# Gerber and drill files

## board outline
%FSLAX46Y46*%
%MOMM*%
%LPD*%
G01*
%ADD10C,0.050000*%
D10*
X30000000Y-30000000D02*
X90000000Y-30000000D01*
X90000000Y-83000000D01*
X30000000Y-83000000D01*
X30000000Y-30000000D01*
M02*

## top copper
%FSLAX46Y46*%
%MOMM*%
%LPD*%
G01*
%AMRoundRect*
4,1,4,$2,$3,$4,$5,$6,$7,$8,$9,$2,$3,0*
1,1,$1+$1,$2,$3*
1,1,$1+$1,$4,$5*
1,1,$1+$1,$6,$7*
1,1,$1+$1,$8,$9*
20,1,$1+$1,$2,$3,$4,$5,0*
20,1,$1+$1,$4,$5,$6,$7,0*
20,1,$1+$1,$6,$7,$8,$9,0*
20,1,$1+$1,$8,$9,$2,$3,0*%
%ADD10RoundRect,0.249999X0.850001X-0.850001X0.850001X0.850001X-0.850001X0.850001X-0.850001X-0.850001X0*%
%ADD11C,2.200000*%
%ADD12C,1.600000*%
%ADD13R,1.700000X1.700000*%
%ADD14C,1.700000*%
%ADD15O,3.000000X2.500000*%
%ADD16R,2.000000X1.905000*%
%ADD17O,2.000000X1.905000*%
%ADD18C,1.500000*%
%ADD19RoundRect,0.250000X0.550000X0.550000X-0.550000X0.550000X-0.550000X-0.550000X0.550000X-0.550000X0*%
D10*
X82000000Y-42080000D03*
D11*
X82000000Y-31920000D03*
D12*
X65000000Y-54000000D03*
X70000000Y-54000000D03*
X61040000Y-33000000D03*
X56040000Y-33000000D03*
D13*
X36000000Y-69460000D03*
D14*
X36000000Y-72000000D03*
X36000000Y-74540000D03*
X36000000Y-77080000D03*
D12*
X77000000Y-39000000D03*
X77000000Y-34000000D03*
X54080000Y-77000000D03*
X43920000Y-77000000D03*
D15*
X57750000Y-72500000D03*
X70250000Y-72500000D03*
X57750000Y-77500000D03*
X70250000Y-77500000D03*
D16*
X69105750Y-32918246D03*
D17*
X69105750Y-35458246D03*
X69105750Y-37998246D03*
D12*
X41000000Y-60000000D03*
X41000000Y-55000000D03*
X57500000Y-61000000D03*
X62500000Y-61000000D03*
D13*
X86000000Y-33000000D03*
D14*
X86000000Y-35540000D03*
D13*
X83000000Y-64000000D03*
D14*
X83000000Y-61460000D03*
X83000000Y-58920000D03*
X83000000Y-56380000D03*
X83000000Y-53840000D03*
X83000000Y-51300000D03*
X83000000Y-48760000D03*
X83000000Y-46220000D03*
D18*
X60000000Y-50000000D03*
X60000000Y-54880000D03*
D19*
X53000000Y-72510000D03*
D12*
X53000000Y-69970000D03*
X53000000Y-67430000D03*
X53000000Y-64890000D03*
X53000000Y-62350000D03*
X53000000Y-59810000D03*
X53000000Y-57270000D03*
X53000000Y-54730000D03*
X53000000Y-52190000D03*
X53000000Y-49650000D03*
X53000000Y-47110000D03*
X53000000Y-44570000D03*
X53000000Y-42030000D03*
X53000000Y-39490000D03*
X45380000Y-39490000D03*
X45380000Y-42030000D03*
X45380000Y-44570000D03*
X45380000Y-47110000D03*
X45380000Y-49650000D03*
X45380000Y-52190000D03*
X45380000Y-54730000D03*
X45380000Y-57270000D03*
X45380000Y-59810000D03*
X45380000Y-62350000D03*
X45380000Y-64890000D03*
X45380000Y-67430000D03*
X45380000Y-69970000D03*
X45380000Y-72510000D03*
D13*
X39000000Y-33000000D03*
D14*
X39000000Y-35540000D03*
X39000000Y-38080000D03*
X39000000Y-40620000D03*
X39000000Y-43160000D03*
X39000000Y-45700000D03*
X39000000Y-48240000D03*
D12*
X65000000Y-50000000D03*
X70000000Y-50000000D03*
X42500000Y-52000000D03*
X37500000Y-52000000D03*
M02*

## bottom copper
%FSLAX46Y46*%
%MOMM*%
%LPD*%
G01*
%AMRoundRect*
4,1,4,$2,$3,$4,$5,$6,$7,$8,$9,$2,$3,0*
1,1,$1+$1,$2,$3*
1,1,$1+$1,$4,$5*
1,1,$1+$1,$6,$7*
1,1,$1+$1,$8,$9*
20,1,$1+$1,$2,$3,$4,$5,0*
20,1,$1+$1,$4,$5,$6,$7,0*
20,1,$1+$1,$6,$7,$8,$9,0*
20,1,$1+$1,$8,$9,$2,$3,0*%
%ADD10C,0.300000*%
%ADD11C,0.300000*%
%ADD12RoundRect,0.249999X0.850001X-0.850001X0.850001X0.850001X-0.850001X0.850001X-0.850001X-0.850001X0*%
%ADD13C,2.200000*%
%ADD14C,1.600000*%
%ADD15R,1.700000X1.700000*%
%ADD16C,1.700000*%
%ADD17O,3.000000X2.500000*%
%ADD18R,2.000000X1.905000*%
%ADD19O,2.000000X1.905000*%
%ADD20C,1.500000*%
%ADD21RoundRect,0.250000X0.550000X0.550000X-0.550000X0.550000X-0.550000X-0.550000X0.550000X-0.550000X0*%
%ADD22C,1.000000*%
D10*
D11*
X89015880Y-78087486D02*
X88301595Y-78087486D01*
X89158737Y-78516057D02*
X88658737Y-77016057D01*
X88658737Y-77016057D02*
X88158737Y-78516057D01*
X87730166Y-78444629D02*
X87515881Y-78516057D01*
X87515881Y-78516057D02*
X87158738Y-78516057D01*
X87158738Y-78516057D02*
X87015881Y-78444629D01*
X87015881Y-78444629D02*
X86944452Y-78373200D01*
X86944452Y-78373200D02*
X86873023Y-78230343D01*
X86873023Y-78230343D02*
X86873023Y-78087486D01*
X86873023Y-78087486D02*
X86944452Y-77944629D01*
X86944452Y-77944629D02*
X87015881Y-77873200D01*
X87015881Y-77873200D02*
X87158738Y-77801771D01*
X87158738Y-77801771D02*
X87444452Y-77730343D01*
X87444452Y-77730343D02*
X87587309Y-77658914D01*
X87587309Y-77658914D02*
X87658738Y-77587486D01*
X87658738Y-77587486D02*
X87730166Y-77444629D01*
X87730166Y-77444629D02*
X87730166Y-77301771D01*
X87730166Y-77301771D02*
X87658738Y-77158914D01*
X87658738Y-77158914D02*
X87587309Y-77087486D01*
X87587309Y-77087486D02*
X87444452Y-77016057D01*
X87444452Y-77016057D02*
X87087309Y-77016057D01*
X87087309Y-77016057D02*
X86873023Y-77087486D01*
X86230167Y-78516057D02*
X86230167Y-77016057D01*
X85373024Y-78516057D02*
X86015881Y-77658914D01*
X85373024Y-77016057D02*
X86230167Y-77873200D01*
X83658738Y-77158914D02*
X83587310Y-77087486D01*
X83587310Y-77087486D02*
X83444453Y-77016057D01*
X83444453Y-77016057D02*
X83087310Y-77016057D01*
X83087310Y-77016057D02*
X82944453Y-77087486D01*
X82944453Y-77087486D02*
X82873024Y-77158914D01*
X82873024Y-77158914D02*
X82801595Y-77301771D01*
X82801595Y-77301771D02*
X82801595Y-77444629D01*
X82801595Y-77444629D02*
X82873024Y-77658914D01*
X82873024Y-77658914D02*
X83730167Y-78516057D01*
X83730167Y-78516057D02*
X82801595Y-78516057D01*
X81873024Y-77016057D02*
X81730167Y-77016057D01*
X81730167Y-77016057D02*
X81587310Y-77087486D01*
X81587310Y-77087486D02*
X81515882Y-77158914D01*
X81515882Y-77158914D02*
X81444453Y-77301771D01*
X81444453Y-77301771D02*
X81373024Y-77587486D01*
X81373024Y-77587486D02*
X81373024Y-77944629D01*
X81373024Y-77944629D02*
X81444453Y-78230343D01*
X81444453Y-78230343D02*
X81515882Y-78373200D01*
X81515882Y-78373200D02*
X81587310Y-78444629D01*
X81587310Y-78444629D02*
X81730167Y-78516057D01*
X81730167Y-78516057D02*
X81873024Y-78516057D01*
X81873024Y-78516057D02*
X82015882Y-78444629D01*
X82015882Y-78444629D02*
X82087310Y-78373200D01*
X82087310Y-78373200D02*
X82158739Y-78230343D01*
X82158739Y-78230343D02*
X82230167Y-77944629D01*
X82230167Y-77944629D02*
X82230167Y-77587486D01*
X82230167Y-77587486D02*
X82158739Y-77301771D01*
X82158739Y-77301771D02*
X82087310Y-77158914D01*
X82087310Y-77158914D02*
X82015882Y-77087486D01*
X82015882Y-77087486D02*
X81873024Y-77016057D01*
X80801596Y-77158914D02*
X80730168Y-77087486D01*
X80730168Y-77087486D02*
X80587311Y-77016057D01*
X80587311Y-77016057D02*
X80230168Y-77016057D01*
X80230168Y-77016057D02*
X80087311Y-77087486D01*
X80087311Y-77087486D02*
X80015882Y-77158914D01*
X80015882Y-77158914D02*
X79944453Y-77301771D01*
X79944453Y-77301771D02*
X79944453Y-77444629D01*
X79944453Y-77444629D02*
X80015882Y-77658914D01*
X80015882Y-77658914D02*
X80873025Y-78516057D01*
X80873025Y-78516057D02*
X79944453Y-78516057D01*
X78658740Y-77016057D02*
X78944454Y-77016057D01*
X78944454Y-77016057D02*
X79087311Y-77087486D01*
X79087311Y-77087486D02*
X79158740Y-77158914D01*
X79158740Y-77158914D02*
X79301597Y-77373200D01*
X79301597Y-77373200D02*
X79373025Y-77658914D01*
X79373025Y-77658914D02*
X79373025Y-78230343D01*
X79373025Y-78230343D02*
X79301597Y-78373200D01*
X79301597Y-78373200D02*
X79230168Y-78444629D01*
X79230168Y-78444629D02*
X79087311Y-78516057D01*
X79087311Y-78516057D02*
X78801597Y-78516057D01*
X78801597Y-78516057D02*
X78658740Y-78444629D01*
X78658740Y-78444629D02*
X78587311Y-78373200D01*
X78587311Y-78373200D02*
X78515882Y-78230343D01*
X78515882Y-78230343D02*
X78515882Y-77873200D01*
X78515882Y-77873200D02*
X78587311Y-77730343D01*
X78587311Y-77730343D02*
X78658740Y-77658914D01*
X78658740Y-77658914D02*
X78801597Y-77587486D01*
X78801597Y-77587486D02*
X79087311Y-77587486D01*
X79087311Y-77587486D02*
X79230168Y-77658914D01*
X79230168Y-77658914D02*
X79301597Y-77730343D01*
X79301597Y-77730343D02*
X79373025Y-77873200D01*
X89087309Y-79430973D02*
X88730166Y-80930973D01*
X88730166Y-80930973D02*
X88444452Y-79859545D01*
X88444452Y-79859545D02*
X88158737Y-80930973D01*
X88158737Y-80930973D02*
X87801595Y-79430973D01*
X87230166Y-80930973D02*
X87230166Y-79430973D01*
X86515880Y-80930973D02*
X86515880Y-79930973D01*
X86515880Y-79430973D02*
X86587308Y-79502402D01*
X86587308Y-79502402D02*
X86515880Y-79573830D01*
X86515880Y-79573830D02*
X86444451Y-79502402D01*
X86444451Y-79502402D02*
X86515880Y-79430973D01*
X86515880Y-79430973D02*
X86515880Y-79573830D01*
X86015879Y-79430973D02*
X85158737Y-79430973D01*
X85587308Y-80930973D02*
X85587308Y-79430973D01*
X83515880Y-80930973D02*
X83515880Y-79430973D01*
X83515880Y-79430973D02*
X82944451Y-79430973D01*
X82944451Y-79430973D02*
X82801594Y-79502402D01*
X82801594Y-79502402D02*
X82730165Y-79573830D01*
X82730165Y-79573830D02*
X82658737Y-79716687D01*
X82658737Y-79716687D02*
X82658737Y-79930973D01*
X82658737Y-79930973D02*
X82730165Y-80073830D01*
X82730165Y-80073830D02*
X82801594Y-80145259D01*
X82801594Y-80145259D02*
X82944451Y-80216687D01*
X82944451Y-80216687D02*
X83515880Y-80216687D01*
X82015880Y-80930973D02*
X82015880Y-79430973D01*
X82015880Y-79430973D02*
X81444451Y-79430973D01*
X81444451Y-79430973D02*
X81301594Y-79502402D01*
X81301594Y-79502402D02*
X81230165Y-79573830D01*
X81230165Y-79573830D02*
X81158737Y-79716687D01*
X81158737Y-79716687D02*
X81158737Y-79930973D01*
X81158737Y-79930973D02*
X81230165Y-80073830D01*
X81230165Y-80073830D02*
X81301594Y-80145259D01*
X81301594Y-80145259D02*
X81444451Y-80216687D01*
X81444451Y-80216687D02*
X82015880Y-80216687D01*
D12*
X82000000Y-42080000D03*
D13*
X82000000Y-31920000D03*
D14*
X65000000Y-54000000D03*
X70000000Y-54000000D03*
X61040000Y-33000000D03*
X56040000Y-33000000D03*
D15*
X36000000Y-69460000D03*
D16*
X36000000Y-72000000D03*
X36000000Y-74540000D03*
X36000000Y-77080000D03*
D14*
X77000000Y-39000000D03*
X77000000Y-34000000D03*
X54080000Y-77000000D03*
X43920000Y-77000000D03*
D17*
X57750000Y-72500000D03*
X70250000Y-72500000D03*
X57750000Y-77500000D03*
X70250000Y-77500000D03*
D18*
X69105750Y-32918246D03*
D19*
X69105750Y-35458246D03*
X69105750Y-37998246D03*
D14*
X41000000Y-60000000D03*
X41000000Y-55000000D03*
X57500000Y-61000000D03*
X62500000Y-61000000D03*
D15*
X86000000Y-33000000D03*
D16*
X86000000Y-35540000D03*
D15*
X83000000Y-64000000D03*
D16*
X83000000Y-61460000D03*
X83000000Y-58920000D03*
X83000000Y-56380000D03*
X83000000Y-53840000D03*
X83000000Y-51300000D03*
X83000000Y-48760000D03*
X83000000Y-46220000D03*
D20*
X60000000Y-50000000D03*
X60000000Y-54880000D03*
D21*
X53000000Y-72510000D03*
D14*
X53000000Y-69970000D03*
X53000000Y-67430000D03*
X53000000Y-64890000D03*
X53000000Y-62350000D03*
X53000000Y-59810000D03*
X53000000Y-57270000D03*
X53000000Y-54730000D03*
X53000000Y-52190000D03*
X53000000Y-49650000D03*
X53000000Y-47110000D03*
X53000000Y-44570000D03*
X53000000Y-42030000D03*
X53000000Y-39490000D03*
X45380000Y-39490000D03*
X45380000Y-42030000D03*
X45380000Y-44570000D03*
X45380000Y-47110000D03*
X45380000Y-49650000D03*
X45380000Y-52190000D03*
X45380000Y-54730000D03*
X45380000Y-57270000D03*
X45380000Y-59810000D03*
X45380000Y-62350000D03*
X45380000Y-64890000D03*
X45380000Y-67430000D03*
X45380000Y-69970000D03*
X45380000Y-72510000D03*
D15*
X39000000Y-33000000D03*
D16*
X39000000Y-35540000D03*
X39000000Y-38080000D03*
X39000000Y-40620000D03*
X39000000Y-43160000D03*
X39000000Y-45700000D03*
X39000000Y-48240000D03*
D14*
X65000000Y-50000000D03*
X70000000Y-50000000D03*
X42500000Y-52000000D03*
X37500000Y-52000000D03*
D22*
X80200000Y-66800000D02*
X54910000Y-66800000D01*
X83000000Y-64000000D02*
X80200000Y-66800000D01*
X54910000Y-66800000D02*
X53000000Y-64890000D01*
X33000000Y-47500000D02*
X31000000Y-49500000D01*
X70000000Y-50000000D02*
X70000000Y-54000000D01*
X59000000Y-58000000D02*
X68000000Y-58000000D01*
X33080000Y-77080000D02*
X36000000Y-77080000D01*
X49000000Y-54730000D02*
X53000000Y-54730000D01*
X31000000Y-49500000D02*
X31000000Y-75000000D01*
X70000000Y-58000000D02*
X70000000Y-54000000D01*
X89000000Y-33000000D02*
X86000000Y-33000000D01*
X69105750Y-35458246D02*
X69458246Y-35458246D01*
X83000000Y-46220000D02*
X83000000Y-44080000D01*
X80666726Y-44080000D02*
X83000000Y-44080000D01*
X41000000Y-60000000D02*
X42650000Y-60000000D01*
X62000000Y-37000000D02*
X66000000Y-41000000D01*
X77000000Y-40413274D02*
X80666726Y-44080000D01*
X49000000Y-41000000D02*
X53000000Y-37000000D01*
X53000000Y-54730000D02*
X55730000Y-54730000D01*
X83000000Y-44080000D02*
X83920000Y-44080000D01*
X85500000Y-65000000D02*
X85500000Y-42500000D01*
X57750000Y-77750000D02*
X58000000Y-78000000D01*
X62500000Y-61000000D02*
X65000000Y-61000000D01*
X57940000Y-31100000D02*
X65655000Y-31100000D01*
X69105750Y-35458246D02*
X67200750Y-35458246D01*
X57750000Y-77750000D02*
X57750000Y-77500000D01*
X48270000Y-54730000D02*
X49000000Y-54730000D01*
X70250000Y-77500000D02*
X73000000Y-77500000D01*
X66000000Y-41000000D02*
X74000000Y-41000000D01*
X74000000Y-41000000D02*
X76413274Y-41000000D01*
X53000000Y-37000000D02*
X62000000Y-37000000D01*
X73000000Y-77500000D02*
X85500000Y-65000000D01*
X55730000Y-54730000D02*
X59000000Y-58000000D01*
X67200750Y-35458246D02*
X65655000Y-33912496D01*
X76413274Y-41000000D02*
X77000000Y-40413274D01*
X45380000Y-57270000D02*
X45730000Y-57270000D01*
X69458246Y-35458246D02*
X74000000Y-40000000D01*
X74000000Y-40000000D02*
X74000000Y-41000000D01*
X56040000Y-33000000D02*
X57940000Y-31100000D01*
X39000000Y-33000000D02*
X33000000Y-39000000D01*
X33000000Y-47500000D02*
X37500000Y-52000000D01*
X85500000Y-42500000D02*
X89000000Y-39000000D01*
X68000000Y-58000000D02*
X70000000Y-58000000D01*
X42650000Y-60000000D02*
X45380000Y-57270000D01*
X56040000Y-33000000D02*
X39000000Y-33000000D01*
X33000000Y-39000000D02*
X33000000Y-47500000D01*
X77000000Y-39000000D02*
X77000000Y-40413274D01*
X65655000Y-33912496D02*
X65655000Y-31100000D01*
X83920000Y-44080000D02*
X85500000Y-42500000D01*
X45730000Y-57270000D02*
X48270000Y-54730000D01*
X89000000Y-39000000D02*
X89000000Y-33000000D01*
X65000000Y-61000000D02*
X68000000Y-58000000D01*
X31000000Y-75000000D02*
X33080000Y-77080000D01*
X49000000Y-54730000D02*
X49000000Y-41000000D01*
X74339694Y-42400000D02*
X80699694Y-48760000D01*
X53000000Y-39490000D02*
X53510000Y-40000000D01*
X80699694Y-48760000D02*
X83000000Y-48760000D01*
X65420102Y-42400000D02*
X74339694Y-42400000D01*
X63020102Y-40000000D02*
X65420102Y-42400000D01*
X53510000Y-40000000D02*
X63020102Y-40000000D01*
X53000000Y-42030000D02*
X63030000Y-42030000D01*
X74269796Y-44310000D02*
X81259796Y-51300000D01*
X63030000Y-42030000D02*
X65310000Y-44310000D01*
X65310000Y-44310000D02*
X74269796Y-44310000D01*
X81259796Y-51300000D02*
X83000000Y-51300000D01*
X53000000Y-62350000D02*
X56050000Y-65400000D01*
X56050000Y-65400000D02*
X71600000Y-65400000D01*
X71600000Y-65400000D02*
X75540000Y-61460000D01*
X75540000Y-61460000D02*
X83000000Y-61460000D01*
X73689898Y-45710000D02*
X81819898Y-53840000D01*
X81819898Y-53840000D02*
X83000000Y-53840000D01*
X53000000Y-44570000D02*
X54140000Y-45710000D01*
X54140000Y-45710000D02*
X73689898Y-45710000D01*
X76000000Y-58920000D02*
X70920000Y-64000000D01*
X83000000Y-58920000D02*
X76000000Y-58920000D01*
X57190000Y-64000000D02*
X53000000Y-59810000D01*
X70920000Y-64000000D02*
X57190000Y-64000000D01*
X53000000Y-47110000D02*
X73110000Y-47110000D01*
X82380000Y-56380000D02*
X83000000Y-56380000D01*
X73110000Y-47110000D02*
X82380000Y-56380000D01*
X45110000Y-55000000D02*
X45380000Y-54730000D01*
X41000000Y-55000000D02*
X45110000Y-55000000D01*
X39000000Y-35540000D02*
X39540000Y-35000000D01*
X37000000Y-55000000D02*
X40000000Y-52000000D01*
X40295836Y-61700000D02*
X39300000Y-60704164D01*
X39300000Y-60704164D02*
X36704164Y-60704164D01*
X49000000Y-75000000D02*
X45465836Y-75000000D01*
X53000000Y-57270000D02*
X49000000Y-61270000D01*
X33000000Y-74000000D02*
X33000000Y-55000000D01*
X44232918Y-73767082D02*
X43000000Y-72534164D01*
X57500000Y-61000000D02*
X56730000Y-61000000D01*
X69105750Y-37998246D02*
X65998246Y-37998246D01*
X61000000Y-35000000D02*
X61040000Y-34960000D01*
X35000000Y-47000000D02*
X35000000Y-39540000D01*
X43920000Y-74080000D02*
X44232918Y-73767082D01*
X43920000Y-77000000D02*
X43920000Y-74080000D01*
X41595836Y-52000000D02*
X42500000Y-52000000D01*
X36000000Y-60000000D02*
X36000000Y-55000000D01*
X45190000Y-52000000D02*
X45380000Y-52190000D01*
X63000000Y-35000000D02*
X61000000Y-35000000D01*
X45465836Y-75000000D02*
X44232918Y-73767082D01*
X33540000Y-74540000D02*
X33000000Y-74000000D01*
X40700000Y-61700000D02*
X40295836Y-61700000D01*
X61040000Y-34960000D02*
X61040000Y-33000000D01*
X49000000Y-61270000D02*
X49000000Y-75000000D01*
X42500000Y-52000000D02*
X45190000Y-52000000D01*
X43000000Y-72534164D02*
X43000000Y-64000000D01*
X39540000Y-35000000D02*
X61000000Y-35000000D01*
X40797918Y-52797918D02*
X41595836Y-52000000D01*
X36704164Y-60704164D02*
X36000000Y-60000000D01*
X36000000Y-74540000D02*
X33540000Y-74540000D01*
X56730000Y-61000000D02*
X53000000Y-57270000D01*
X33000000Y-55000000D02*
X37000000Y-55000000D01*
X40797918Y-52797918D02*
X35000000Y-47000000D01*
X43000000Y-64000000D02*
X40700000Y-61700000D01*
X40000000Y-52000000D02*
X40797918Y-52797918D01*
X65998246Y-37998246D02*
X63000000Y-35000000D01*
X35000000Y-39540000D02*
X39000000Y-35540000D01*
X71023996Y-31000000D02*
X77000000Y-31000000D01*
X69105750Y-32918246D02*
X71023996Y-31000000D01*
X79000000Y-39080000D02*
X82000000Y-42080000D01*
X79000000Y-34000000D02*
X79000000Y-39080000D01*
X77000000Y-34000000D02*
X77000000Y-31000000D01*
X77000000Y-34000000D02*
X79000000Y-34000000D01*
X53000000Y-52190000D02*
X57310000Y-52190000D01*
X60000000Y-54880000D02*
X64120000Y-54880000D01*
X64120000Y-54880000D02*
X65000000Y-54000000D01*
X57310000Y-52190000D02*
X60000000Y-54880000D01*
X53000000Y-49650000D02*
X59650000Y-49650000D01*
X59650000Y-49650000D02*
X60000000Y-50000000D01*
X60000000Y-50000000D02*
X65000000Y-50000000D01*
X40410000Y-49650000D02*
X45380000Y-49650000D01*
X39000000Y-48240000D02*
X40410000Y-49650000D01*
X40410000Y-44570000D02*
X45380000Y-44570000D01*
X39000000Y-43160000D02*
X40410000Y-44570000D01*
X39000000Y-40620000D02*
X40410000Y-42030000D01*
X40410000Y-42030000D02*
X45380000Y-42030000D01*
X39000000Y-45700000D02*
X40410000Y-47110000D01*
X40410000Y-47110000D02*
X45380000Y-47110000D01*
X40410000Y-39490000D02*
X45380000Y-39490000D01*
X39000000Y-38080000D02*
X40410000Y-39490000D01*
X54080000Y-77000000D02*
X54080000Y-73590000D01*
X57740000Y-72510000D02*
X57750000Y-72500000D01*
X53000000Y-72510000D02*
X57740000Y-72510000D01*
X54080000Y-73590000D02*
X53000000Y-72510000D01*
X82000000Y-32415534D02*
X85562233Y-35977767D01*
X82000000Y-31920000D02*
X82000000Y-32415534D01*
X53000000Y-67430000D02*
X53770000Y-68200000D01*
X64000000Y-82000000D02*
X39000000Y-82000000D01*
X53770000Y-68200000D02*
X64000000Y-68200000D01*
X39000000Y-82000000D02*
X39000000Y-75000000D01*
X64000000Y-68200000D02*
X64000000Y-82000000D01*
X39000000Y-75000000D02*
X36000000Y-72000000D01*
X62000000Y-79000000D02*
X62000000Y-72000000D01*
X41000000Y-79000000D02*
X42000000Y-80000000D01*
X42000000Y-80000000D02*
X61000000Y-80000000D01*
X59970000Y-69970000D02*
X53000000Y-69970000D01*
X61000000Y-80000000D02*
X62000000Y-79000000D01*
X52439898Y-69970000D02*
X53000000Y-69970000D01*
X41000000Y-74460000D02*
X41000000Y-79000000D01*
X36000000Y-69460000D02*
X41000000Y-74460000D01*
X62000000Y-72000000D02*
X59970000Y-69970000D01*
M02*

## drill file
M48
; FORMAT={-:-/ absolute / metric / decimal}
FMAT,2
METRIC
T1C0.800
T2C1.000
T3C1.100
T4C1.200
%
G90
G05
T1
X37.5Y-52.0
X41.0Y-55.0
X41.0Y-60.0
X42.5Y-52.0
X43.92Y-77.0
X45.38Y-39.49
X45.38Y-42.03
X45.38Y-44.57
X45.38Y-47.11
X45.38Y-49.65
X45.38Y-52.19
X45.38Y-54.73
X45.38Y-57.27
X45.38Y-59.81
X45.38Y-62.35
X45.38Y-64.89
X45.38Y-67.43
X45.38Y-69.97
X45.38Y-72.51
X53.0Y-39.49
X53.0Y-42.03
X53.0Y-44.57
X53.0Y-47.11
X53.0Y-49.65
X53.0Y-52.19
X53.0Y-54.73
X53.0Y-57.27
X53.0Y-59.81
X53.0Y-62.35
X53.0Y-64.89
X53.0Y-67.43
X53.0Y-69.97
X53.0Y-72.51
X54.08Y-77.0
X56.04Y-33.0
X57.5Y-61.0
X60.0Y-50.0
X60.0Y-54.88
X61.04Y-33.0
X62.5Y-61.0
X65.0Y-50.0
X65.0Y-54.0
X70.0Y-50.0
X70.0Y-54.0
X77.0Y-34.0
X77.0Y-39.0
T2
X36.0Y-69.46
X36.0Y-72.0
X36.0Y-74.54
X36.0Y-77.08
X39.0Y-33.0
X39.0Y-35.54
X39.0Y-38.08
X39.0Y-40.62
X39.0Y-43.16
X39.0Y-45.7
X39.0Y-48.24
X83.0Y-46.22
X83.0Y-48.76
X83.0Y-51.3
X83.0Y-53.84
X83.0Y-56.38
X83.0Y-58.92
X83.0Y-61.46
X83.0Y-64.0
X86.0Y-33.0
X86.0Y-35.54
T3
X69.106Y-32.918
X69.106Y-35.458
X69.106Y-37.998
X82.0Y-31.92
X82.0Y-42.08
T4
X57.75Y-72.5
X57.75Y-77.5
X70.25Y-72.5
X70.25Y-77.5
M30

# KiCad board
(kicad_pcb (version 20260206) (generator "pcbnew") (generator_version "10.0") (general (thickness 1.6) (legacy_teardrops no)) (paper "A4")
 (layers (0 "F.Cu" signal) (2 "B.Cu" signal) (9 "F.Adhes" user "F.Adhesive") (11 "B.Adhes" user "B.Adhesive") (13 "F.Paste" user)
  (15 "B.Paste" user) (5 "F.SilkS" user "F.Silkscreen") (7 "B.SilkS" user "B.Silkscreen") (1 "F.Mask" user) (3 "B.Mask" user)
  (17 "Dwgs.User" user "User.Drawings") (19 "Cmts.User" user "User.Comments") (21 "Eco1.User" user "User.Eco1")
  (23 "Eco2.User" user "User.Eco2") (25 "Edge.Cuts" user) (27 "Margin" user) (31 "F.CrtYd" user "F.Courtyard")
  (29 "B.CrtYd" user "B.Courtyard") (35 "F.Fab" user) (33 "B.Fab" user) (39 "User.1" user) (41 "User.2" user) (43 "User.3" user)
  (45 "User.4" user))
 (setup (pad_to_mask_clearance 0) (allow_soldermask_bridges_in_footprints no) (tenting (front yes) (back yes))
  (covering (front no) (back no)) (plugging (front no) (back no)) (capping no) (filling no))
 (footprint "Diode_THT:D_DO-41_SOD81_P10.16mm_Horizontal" (layer "F.Cu") (at 82 42.08 90)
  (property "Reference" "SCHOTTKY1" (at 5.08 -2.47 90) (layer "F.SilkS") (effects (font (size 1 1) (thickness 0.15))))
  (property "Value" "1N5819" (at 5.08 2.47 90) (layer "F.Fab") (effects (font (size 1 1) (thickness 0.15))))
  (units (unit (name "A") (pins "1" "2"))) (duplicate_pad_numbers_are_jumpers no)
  (pad "1" thru_hole roundrect (at 0 0 90) (size 2.2 2.2) (drill 1.1) (layers "*.Cu" "*.Mask") (remove_unused_layers no)
   (roundrect_rratio 0.113636) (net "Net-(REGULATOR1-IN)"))
  (pad "2" thru_hole circle (at 10.16 0 90) (size 2.2 2.2) (drill 1.1) (layers "*.Cu" "*.Mask") (remove_unused_layers no)
   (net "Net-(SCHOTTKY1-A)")))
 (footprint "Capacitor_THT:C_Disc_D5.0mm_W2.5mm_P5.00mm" (layer "F.Cu") (at 65 54)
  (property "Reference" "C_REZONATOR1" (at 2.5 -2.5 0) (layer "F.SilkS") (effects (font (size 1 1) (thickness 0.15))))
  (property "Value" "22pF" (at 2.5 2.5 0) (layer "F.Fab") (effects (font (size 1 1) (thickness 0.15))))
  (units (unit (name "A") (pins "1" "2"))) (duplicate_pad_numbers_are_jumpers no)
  (pad "1" thru_hole circle (at 0 0) (size 1.6 1.6) (drill 0.8) (layers "*.Cu" "*.Mask") (remove_unused_layers no)
   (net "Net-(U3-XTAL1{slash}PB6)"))
  (pad "2" thru_hole circle (at 5 0) (size 1.6 1.6) (drill 0.8) (layers "*.Cu" "*.Mask") (remove_unused_layers no) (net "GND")))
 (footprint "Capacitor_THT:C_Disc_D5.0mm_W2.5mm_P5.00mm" (layer "F.Cu") (at 61.04 33 180)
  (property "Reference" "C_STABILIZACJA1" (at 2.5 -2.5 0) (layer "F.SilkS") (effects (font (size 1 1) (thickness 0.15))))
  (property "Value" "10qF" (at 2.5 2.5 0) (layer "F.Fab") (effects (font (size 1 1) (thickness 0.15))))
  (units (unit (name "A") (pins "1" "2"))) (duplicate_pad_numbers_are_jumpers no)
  (pad "1" thru_hole circle (at 0 0 180) (size 1.6 1.6) (drill 0.8) (layers "*.Cu" "*.Mask") (remove_unused_layers no) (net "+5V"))
  (pad "2" thru_hole circle (at 5 0 180) (size 1.6 1.6) (drill 0.8) (layers "*.Cu" "*.Mask") (remove_unused_layers no) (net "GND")))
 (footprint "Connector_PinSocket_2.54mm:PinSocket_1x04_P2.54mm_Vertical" (layer "F.Cu") (at 36 69.46)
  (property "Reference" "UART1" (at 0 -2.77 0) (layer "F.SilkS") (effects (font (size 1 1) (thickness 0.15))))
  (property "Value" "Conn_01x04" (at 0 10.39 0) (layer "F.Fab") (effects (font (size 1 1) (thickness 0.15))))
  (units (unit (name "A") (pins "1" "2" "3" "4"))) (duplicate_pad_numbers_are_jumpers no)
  (pad "1" thru_hole rect (at 0 0) (size 1.7 1.7) (drill 1) (layers "*.Cu" "*.Mask") (remove_unused_layers no) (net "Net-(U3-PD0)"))
  (pad "2" thru_hole circle (at 0 2.54) (size 1.7 1.7) (drill 1) (layers "*.Cu" "*.Mask") (remove_unused_layers no) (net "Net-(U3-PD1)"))
  (pad "3" thru_hole circle (at 0 5.08) (size 1.7 1.7) (drill 1) (layers "*.Cu" "*.Mask") (remove_unused_layers no) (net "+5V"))
  (pad "4" thru_hole circle (at 0 7.62) (size 1.7 1.7) (drill 1) (layers "*.Cu" "*.Mask") (remove_unused_layers no) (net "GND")))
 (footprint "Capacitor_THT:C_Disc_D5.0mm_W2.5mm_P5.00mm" (layer "F.Cu") (at 77 39 90)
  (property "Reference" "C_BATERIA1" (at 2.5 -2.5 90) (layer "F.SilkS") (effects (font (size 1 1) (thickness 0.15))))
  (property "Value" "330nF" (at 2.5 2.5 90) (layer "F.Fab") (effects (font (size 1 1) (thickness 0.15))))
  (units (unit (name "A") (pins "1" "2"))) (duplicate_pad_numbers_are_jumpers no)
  (pad "1" thru_hole circle (at 0 0 90) (size 1.6 1.6) (drill 0.8) (layers "*.Cu" "*.Mask") (remove_unused_layers no) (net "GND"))
  (pad "2" thru_hole circle (at 5 0 90) (size 1.6 1.6) (drill 0.8) (layers "*.Cu" "*.Mask") (remove_unused_layers no)
   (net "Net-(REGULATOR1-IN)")))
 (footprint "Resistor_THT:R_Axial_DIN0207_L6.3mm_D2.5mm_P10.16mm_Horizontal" (layer "F.Cu") (at 54.08 77 180)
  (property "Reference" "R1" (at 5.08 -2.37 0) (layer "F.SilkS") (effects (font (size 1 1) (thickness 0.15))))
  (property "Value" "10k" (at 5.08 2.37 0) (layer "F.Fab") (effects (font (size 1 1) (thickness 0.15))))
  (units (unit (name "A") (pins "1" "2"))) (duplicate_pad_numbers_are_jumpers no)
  (pad "1" thru_hole circle (at 0 0 180) (size 1.6 1.6) (drill 0.8) (layers "*.Cu" "*.Mask") (remove_unused_layers no)
   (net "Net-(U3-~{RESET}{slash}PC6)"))
  (pad "2" thru_hole circle (at 10.16 0 180) (size 1.6 1.6) (drill 0.8) (layers "*.Cu" "*.Mask") (remove_unused_layers no) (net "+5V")))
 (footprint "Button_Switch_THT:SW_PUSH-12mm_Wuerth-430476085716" (layer "F.Cu") (at 57.75 72.5)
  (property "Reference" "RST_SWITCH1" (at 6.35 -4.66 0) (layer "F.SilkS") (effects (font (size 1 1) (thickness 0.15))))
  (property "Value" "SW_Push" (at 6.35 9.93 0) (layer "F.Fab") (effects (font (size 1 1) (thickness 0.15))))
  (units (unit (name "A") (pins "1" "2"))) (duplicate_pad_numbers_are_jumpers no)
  (pad "1" thru_hole oval (at 0 0) (size 3 2.5) (drill 1.2) (layers "*.Cu" "*.Mask") (remove_unused_layers no)
   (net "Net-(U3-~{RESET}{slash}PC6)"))
  (pad "1" thru_hole oval (at 12.5 0) (size 3 2.5) (drill 1.2) (layers "*.Cu" "*.Mask") (remove_unused_layers no)
   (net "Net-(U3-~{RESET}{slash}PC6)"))
  (pad "2" thru_hole oval (at 0 5) (size 3 2.5) (drill 1.2) (layers "*.Cu" "*.Mask") (remove_unused_layers no) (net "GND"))
  (pad "2" thru_hole oval (at 12.5 5) (size 3 2.5) (drill 1.2) (layers "*.Cu" "*.Mask") (remove_unused_layers no) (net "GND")))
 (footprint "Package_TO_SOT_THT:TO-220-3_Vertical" (layer "F.Cu") (at 69.10575 32.918246 -90)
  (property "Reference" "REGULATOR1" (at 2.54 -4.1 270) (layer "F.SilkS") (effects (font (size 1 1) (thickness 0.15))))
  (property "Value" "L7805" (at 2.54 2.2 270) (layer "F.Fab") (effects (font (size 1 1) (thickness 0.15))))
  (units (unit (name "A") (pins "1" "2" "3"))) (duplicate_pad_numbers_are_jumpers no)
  (pad "1" thru_hole rect (at 0 0 270) (size 1.905 2) (drill 1.1) (layers "*.Cu" "*.Mask") (remove_unused_layers no)
   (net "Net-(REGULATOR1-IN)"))
  (pad "2" thru_hole oval (at 2.54 0 270) (size 1.905 2) (drill 1.1) (layers "*.Cu" "*.Mask") (remove_unused_layers no) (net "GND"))
  (pad "3" thru_hole oval (at 5.08 0 270) (size 1.905 2) (drill 1.1) (layers "*.Cu" "*.Mask") (remove_unused_layers no) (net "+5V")))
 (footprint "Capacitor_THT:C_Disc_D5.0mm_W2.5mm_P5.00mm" (layer "F.Cu") (at 41 60 90)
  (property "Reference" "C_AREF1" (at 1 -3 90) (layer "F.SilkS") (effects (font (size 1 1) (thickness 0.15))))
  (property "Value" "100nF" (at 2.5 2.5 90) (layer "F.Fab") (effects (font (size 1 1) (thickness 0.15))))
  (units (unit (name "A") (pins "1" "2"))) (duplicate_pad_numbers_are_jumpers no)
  (pad "1" thru_hole circle (at 0 0 90) (size 1.6 1.6) (drill 0.8) (layers "*.Cu" "*.Mask") (remove_unused_layers no) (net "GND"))
  (pad "2" thru_hole circle (at 5 0 90) (size 1.6 1.6) (drill 0.8) (layers "*.Cu" "*.Mask") (remove_unused_layers no) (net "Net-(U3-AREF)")))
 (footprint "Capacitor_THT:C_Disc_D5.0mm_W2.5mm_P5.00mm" (layer "F.Cu") (at 57.5 61)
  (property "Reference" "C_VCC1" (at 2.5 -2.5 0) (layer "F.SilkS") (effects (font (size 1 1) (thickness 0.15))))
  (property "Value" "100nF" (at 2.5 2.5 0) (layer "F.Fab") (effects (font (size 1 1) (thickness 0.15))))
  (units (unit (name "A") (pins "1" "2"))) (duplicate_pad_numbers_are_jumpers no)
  (pad "1" thru_hole circle (at 0 0) (size 1.6 1.6) (drill 0.8) (layers "*.Cu" "*.Mask") (remove_unused_layers no) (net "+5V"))
  (pad "2" thru_hole circle (at 5 0) (size 1.6 1.6) (drill 0.8) (layers "*.Cu" "*.Mask") (remove_unused_layers no) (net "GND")))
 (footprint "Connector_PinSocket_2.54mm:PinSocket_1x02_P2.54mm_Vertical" (layer "F.Cu") (at 86 33)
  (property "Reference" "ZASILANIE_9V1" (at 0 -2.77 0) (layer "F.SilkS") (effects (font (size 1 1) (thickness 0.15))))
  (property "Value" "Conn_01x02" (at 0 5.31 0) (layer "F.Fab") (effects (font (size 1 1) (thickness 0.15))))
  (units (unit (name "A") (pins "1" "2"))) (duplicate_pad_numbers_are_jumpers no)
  (pad "1" thru_hole rect (at 0 0) (size 1.7 1.7) (drill 1) (layers "*.Cu" "*.Mask") (remove_unused_layers no) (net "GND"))
  (pad "2" thru_hole circle (at 0 2.54) (size 1.7 1.7) (drill 1) (layers "*.Cu" "*.Mask") (remove_unused_layers no)
   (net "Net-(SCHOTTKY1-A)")))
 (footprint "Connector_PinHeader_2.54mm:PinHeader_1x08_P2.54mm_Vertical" (layer "F.Cu") (at 83 64 180)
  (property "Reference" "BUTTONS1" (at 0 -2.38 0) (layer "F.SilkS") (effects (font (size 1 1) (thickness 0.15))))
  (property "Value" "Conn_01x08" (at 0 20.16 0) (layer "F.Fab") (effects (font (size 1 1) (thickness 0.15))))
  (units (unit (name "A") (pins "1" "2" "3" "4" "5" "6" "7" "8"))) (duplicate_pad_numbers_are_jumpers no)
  (pad "1" thru_hole rect (at 0 0 180) (size 1.7 1.7) (drill 1) (layers "*.Cu" "*.Mask") (remove_unused_layers no)
   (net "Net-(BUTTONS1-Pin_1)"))
  (pad "2" thru_hole circle (at 0 2.54 180) (size 1.7 1.7) (drill 1) (layers "*.Cu" "*.Mask") (remove_unused_layers no)
   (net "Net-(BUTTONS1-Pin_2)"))
  (pad "3" thru_hole circle (at 0 5.08 180) (size 1.7 1.7) (drill 1) (layers "*.Cu" "*.Mask") (remove_unused_layers no)
   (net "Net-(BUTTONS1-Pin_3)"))
  (pad "4" thru_hole circle (at 0 7.62 180) (size 1.7 1.7) (drill 1) (layers "*.Cu" "*.Mask") (remove_unused_layers no)
   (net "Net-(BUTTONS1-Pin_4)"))
  (pad "5" thru_hole circle (at 0 10.16 180) (size 1.7 1.7) (drill 1) (layers "*.Cu" "*.Mask") (remove_unused_layers no)
   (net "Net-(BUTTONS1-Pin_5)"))
  (pad "6" thru_hole circle (at 0 12.7 180) (size 1.7 1.7) (drill 1) (layers "*.Cu" "*.Mask") (remove_unused_layers no)
   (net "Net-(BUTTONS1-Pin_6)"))
  (pad "7" thru_hole circle (at 0 15.24 180) (size 1.7 1.7) (drill 1) (layers "*.Cu" "*.Mask") (remove_unused_layers no)
   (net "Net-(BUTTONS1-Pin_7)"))
  (pad "8" thru_hole circle (at 0 17.78 180) (size 1.7 1.7) (drill 1) (layers "*.Cu" "*.Mask") (remove_unused_layers no) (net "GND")))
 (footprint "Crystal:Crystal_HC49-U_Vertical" (layer "F.Cu") (at 60 50 -90)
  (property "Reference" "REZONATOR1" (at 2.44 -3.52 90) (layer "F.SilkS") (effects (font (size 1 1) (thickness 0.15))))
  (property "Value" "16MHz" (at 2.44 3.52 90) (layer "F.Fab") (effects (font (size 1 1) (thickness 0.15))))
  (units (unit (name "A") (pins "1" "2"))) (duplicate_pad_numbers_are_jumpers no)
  (pad "1" thru_hole circle (at 0 0 270) (size 1.5 1.5) (drill 0.8) (layers "*.Cu" "*.Mask") (remove_unused_layers no)
   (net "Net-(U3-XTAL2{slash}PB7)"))
  (pad "2" thru_hole circle (at 4.88 0 270) (size 1.5 1.5) (drill 0.8) (layers "*.Cu" "*.Mask") (remove_unused_layers no)
   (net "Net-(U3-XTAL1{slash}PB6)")))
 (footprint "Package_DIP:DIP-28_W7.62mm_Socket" (layer "F.Cu") (at 53 72.51 180)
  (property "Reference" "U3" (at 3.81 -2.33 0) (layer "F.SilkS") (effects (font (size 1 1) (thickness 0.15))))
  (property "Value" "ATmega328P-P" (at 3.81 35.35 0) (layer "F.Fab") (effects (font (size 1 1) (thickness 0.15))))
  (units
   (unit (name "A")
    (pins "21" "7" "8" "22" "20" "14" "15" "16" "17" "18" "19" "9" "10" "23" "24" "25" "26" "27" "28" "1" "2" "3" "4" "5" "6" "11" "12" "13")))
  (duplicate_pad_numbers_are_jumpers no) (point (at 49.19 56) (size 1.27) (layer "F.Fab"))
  (pad "1" thru_hole roundrect (at 0 0 180) (size 1.6 1.6) (drill 0.8) (layers "*.Cu" "*.Mask") (remove_unused_layers no)
   (roundrect_rratio 0.15625) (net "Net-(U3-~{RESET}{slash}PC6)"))
  (pad "2" thru_hole circle (at 0 2.54 180) (size 1.6 1.6) (drill 0.8) (layers "*.Cu" "*.Mask") (remove_unused_layers no)
   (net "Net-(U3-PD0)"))
  (pad "3" thru_hole circle (at 0 5.08 180) (size 1.6 1.6) (drill 0.8) (layers "*.Cu" "*.Mask") (remove_unused_layers no)
   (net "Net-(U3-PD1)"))
  (pad "4" thru_hole circle (at 0 7.62 180) (size 1.6 1.6) (drill 0.8) (layers "*.Cu" "*.Mask") (remove_unused_layers no)
   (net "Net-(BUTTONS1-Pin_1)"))
  (pad "5" thru_hole circle (at 0 10.16 180) (size 1.6 1.6) (drill 0.8) (layers "*.Cu" "*.Mask") (remove_unused_layers no)
   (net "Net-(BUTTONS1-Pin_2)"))
  (pad "6" thru_hole circle (at 0 12.7 180) (size 1.6 1.6) (drill 0.8) (layers "*.Cu" "*.Mask") (remove_unused_layers no)
   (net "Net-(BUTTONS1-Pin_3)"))
  (pad "7" thru_hole circle (at 0 15.24 180) (size 1.6 1.6) (drill 0.8) (layers "*.Cu" "*.Mask") (remove_unused_layers no) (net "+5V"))
  (pad "8" thru_hole circle (at 0 17.78 180) (size 1.6 1.6) (drill 0.8) (layers "*.Cu" "*.Mask") (remove_unused_layers no) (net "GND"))
  (pad "9" thru_hole circle (at 0 20.32 180) (size 1.6 1.6) (drill 0.8) (layers "*.Cu" "*.Mask") (remove_unused_layers no)
   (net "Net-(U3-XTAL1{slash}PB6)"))
  (pad "10" thru_hole circle (at 0 22.86 180) (size 1.6 1.6) (drill 0.8) (layers "*.Cu" "*.Mask") (remove_unused_layers no)
   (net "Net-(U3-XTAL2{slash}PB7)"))
  (pad "11" thru_hole circle (at 0 25.4 180) (size 1.6 1.6) (drill 0.8) (layers "*.Cu" "*.Mask") (remove_unused_layers no)
   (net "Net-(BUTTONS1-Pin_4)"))
  (pad "12" thru_hole circle (at 0 27.94 180) (size 1.6 1.6) (drill 0.8) (layers "*.Cu" "*.Mask") (remove_unused_layers no)
   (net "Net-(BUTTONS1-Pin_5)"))
  (pad "13" thru_hole circle (at 0 30.48 180) (size 1.6 1.6) (drill 0.8) (layers "*.Cu" "*.Mask") (remove_unused_layers no)
   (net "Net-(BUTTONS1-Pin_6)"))
  (pad "14" thru_hole circle (at 0 33.02 180) (size 1.6 1.6) (drill 0.8) (layers "*.Cu" "*.Mask") (remove_unused_layers no)
   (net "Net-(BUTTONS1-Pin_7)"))
  (pad "15" thru_hole circle (at 7.62 33.02 180) (size 1.6 1.6) (drill 0.8) (layers "*.Cu" "*.Mask") (remove_unused_layers no)
   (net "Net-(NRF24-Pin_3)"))
  (pad "16" thru_hole circle (at 7.62 30.48 180) (size 1.6 1.6) (drill 0.8) (layers "*.Cu" "*.Mask") (remove_unused_layers no)
   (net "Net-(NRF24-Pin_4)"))
  (pad "17" thru_hole circle (at 7.62 27.94 180) (size 1.6 1.6) (drill 0.8) (layers "*.Cu" "*.Mask") (remove_unused_layers no)
   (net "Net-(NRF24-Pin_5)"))
  (pad "18" thru_hole circle (at 7.62 25.4 180) (size 1.6 1.6) (drill 0.8) (layers "*.Cu" "*.Mask") (remove_unused_layers no)
   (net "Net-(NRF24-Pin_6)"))
  (pad "19" thru_hole circle (at 7.62 22.86 180) (size 1.6 1.6) (drill 0.8) (layers "*.Cu" "*.Mask") (remove_unused_layers no)
   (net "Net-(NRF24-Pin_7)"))
  (pad "20" thru_hole circle (at 7.62 20.32 180) (size 1.6 1.6) (drill 0.8) (layers "*.Cu" "*.Mask") (remove_unused_layers no) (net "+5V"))
  (pad "21" thru_hole circle (at 7.62 17.78 180) (size 1.6 1.6) (drill 0.8) (layers "*.Cu" "*.Mask") (remove_unused_layers no)
   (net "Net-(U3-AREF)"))
  (pad "22" thru_hole circle (at 7.62 15.24 180) (size 1.6 1.6) (drill 0.8) (layers "*.Cu" "*.Mask") (remove_unused_layers no) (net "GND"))
  (pad "23" thru_hole circle (at 7.62 12.7 180) (size 1.6 1.6) (drill 0.8) (layers "*.Cu" "*.Mask") (remove_unused_layers no)
   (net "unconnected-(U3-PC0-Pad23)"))
  (pad "24" thru_hole circle (at 7.62 10.16 180) (size 1.6 1.6) (drill 0.8) (layers "*.Cu" "*.Mask") (remove_unused_layers no)
   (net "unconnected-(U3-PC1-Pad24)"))
  (pad "25" thru_hole circle (at 7.62 7.62 180) (size 1.6 1.6) (drill 0.8) (layers "*.Cu" "*.Mask") (remove_unused_layers no)
   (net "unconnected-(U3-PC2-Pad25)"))
  (pad "26" thru_hole circle (at 7.62 5.08 180) (size 1.6 1.6) (drill 0.8) (layers "*.Cu" "*.Mask") (remove_unused_layers no)
   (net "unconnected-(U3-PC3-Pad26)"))
  (pad "27" thru_hole circle (at 7.62 2.54 180) (size 1.6 1.6) (drill 0.8) (layers "*.Cu" "*.Mask") (remove_unused_layers no)
   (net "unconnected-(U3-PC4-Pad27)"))
  (pad "28" thru_hole circle (at 7.62 0 180) (size 1.6 1.6) (drill 0.8) (layers "*.Cu" "*.Mask") (remove_unused_layers no)
   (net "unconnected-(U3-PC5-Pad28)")))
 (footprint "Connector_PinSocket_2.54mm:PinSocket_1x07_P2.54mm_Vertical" (layer "F.Cu") (at 39 33)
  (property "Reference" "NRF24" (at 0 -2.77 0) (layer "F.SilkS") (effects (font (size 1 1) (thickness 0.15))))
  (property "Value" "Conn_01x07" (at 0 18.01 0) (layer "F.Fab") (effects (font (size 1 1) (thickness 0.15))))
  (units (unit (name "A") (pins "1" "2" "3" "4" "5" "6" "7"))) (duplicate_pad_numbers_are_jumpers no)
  (pad "1" thru_hole rect (at 0 0) (size 1.7 1.7) (drill 1) (layers "*.Cu" "*.Mask") (remove_unused_layers no) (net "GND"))
  (pad "2" thru_hole circle (at 0 2.54) (size 1.7 1.7) (drill 1) (layers "*.Cu" "*.Mask") (remove_unused_layers no) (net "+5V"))
  (pad "3" thru_hole circle (at 0 5.08) (size 1.7 1.7) (drill 1) (layers "*.Cu" "*.Mask") (remove_unused_layers no)
   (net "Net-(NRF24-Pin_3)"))
  (pad "4" thru_hole circle (at 0 7.62) (size 1.7 1.7) (drill 1) (layers "*.Cu" "*.Mask") (remove_unused_layers no)
   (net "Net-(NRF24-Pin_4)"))
  (pad "5" thru_hole circle (at 0 10.16) (size 1.7 1.7) (drill 1) (layers "*.Cu" "*.Mask") (remove_unused_layers no)
   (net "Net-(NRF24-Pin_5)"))
  (pad "6" thru_hole circle (at 0 12.7) (size 1.7 1.7) (drill 1) (layers "*.Cu" "*.Mask") (remove_unused_layers no)
   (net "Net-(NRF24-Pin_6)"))
  (pad "7" thru_hole circle (at 0 15.24) (size 1.7 1.7) (drill 1) (layers "*.Cu" "*.Mask") (remove_unused_layers no)
   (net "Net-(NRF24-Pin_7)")))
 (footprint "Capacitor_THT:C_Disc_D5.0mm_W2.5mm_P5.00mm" (layer "F.Cu") (at 65 50)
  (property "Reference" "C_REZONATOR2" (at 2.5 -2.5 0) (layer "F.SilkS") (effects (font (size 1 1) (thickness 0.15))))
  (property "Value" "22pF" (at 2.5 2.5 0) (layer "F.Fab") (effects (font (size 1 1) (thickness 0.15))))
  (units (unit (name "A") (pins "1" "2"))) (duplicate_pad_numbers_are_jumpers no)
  (pad "1" thru_hole circle (at 0 0) (size 1.6 1.6) (drill 0.8) (layers "*.Cu" "*.Mask") (remove_unused_layers no)
   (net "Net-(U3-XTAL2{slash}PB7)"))
  (pad "2" thru_hole circle (at 5 0) (size 1.6 1.6) (drill 0.8) (layers "*.Cu" "*.Mask") (remove_unused_layers no) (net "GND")))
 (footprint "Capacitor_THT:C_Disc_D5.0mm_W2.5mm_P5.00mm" (layer "F.Cu") (at 42.5 52 180)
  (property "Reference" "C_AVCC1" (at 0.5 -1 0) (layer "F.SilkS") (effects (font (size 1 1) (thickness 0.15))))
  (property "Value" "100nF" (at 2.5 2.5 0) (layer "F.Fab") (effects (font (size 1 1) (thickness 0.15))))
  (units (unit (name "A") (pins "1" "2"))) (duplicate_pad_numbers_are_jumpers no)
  (pad "1" thru_hole circle (at 0 0 180) (size 1.6 1.6) (drill 0.8) (layers "*.Cu" "*.Mask") (remove_unused_layers no) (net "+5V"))
  (pad "2" thru_hole circle (at 5 0 180) (size 1.6 1.6) (drill 0.8) (layers "*.Cu" "*.Mask") (remove_unused_layers no) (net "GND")))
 (gr_rect (start 30 30) (end 90 83) (stroke (width 0.05) (type default)) (fill no) (layer "Edge.Cuts"))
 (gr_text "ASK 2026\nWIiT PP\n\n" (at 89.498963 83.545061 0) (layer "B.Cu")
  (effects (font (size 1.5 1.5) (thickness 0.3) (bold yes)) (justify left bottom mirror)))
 (segment (start 80.2 66.8) (end 54.91 66.8) (width 1) (layer "B.Cu") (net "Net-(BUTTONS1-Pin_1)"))
 (segment (start 83 64) (end 80.2 66.8) (width 1) (layer "B.Cu") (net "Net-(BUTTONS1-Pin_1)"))
 (segment (start 54.91 66.8) (end 53 64.89) (width 1) (layer "B.Cu") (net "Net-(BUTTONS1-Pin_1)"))
 (segment (start 33 47.5) (end 31 49.5) (width 1) (layer "B.Cu") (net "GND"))
 (segment (start 70 50) (end 70 54) (width 1) (layer "B.Cu") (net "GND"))
 (segment (start 59 58) (end 68 58) (width 1) (layer "B.Cu") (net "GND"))
 (segment (start 33.08 77.08) (end 36 77.08) (width 1) (layer "B.Cu") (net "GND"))
 (segment (start 49 54.73) (end 53 54.73) (width 1) (layer "B.Cu") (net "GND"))
 (segment (start 31 49.5) (end 31 75) (width 1) (layer "B.Cu") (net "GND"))
 (segment (start 70 58) (end 70 54) (width 1) (layer "B.Cu") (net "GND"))
 (segment (start 89 33) (end 86 33) (width 1) (layer "B.Cu") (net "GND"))
 (segment (start 69.10575 35.458246) (end 69.458246 35.458246) (width 1) (layer "B.Cu") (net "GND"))
 (segment (start 83 46.22) (end 83 44.08) (width 1) (layer "B.Cu") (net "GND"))
 (segment (start 80.666726 44.08) (end 83 44.08) (width 1) (layer "B.Cu") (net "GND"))
 (segment (start 41 60) (end 42.65 60) (width 1) (layer "B.Cu") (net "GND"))
 (segment (start 62 37) (end 66 41) (width 1) (layer "B.Cu") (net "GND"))
 (segment (start 77 40.413274) (end 80.666726 44.08) (width 1) (layer "B.Cu") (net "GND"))
 (segment (start 49 41) (end 53 37) (width 1) (layer "B.Cu") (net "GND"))
 (segment (start 53 54.73) (end 55.73 54.73) (width 1) (layer "B.Cu") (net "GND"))
 (segment (start 83 44.08) (end 83.92 44.08) (width 1) (layer "B.Cu") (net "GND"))
 (segment (start 85.5 65) (end 85.5 42.5) (width 1) (layer "B.Cu") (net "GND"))
 (segment (start 57.75 77.75) (end 58 78) (width 1) (layer "B.Cu") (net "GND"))
 (segment (start 62.5 61) (end 65 61) (width 1) (layer "B.Cu") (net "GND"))
 (segment (start 57.94 31.1) (end 65.655 31.1) (width 1) (layer "B.Cu") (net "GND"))
 (segment (start 69.10575 35.458246) (end 67.20075 35.458246) (width 1) (layer "B.Cu") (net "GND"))
 (segment (start 57.75 77.75) (end 57.75 77.5) (width 1) (layer "B.Cu") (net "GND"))
 (segment (start 48.27 54.73) (end 49 54.73) (width 1) (layer "B.Cu") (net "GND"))
 (segment (start 70.25 77.5) (end 73 77.5) (width 1) (layer "B.Cu") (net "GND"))
 (segment (start 66 41) (end 74 41) (width 1) (layer "B.Cu") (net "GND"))
 (segment (start 74 41) (end 76.413274 41) (width 1) (layer "B.Cu") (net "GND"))
 (segment (start 53 37) (end 62 37) (width 1) (layer "B.Cu") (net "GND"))
 (segment (start 73 77.5) (end 85.5 65) (width 1) (layer "B.Cu") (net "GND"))
 (segment (start 55.73 54.73) (end 59 58) (width 1) (layer "B.Cu") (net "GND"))
 (segment (start 67.20075 35.458246) (end 65.655 33.912496) (width 1) (layer "B.Cu") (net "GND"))
 (segment (start 76.413274 41) (end 77 40.413274) (width 1) (layer "B.Cu") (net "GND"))
 (segment (start 45.38 57.27) (end 45.73 57.27) (width 1) (layer "B.Cu") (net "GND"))
 (segment (start 69.458246 35.458246) (end 74 40) (width 1) (layer "B.Cu") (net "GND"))
 (segment (start 74 40) (end 74 41) (width 1) (layer "B.Cu") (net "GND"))
 (segment (start 56.04 33) (end 57.94 31.1) (width 1) (layer "B.Cu") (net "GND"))
 (segment (start 39 33) (end 33 39) (width 1) (layer "B.Cu") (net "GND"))
 (segment (start 33 47.5) (end 37.5 52) (width 1) (layer "B.Cu") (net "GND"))
 (segment (start 85.5 42.5) (end 89 39) (width 1) (layer "B.Cu") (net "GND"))
 (segment (start 68 58) (end 70 58) (width 1) (layer "B.Cu") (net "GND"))
 (segment (start 42.65 60) (end 45.38 57.27) (width 1) (layer "B.Cu") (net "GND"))
 (segment (start 56.04 33) (end 39 33) (width 1) (layer "B.Cu") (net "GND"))
 (segment (start 33 39) (end 33 47.5) (width 1) (layer "B.Cu") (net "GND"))
 (segment (start 77 39) (end 77 40.413274) (width 1) (layer "B.Cu") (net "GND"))
 (segment (start 65.655 33.912496) (end 65.655 31.1) (width 1) (layer "B.Cu") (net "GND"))
 (segment (start 83.92 44.08) (end 85.5 42.5) (width 1) (layer "B.Cu") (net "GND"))
 (segment (start 45.73 57.27) (end 48.27 54.73) (width 1) (layer "B.Cu") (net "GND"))
 (segment (start 89 39) (end 89 33) (width 1) (layer "B.Cu") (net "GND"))
 (segment (start 65 61) (end 68 58) (width 1) (layer "B.Cu") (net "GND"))
 (segment (start 31 75) (end 33.08 77.08) (width 1) (layer "B.Cu") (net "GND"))
 (segment (start 49 54.73) (end 49 41) (width 1) (layer "B.Cu") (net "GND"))
 (segment (start 74.339694 42.4) (end 80.699694 48.76) (width 1) (layer "B.Cu") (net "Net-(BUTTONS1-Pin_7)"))
 (segment (start 53 39.49) (end 53.51 40) (width 1) (layer "B.Cu") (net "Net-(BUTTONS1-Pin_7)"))
 (segment (start 80.699694 48.76) (end 83 48.76) (width 1) (layer "B.Cu") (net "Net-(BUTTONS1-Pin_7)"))
 (segment (start 65.420102 42.4) (end 74.339694 42.4) (width 1) (layer "B.Cu") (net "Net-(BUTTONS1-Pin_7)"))
 (segment (start 63.020102 40) (end 65.420102 42.4) (width 1) (layer "B.Cu") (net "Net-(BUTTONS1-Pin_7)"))
 (segment (start 53.51 40) (end 63.020102 40) (width 1) (layer "B.Cu") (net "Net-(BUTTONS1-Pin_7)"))
 (segment (start 53 42.03) (end 63.03 42.03) (width 1) (layer "B.Cu") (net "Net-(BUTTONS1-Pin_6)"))
 (segment (start 74.269796 44.31) (end 81.259796 51.3) (width 1) (layer "B.Cu") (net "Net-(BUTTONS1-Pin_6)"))
 (segment (start 63.03 42.03) (end 65.31 44.31) (width 1) (layer "B.Cu") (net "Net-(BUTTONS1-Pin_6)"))
 (segment (start 65.31 44.31) (end 74.269796 44.31) (width 1) (layer "B.Cu") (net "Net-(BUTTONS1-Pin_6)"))
 (segment (start 81.259796 51.3) (end 83 51.3) (width 1) (layer "B.Cu") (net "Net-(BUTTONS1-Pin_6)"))
 (segment (start 53 62.35) (end 56.05 65.4) (width 1) (layer "B.Cu") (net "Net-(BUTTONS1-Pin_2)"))
 (segment (start 56.05 65.4) (end 71.6 65.4) (width 1) (layer "B.Cu") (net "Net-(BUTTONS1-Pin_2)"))
 (segment (start 71.6 65.4) (end 75.54 61.46) (width 1) (layer "B.Cu") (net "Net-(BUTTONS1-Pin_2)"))
 (segment (start 75.54 61.46) (end 83 61.46) (width 1) (layer "B.Cu") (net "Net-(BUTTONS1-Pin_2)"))
 (segment (start 73.689898 45.71) (end 81.819898 53.84) (width 1) (layer "B.Cu") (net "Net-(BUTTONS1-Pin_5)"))
 (segment (start 81.819898 53.84) (end 83 53.84) (width 1) (layer "B.Cu") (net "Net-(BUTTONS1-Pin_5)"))
 (segment (start 53 44.57) (end 54.14 45.71) (width 1) (layer "B.Cu") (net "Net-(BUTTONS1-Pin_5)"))
 (segment (start 54.14 45.71) (end 73.689898 45.71) (width 1) (layer "B.Cu") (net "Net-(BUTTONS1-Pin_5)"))
 (segment (start 76 58.92) (end 70.92 64) (width 1) (layer "B.Cu") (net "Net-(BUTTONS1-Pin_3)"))
 (segment (start 83 58.92) (end 76 58.92) (width 1) (layer "B.Cu") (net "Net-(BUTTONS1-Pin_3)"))
 (segment (start 57.19 64) (end 53 59.81) (width 1) (layer "B.Cu") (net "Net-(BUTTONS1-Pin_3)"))
 (segment (start 70.92 64) (end 57.19 64) (width 1) (layer "B.Cu") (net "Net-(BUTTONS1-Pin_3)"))
 (segment (start 53 47.11) (end 73.11 47.11) (width 1) (layer "B.Cu") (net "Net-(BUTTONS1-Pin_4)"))
 (segment (start 82.38 56.38) (end 83 56.38) (width 1) (layer "B.Cu") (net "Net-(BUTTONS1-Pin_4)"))
 (segment (start 73.11 47.11) (end 82.38 56.38) (width 1) (layer "B.Cu") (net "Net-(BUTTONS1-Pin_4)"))
 (segment (start 45.11 55) (end 45.38 54.73) (width 1) (layer "B.Cu") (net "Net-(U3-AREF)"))
 (segment (start 41 55) (end 45.11 55) (width 1) (layer "B.Cu") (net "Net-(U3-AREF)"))
 (segment (start 39 35.54) (end 39.54 35) (width 1) (layer "B.Cu") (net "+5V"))
 (segment (start 37 55) (end 40 52) (width 1) (layer "B.Cu") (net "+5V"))
 (segment (start 40.295836 61.7) (end 39.3 60.704164) (width 1) (layer "B.Cu") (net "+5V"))
 (segment (start 39.3 60.704164) (end 36.704164 60.704164) (width 1) (layer "B.Cu") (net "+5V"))
 (segment (start 49 75) (end 45.465836 75) (width 1) (layer "B.Cu") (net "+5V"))
 (segment (start 53 57.27) (end 49 61.27) (width 1) (layer "B.Cu") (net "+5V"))
 (segment (start 33 74) (end 33 55) (width 1) (layer "B.Cu") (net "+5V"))
 (segment (start 44.232918 73.767082) (end 43 72.534164) (width 1) (layer "B.Cu") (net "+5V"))
 (segment (start 57.5 61) (end 56.73 61) (width 1) (layer "B.Cu") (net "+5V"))
 (segment (start 69.10575 37.998246) (end 65.998246 37.998246) (width 1) (layer "B.Cu") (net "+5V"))
 (segment (start 61 35) (end 61.04 34.96) (width 1) (layer "B.Cu") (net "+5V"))
 (segment (start 35 47) (end 35 39.54) (width 1) (layer "B.Cu") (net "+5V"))
 (segment (start 43.92 74.08) (end 44.232918 73.767082) (width 1) (layer "B.Cu") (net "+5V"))
 (segment (start 43.92 77) (end 43.92 74.08) (width 1) (layer "B.Cu") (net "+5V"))
 (segment (start 41.595836 52) (end 42.5 52) (width 1) (layer "B.Cu") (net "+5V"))
 (segment (start 36 60) (end 36 55) (width 1) (layer "B.Cu") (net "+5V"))
 (segment (start 45.19 52) (end 45.38 52.19) (width 1) (layer "B.Cu") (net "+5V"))
 (segment (start 63 35) (end 61 35) (width 1) (layer "B.Cu") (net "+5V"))
 (segment (start 45.465836 75) (end 44.232918 73.767082) (width 1) (layer "B.Cu") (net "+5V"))
 (segment (start 33.54 74.54) (end 33 74) (width 1) (layer "B.Cu") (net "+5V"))
 (segment (start 40.7 61.7) (end 40.295836 61.7) (width 1) (layer "B.Cu") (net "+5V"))
 (segment (start 61.04 34.96) (end 61.04 33) (width 1) (layer "B.Cu") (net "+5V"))
 (segment (start 49 61.27) (end 49 75) (width 1) (layer "B.Cu") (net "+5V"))
 (segment (start 42.5 52) (end 45.19 52) (width 1) (layer "B.Cu") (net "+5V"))
 (segment (start 43 72.534164) (end 43 64) (width 1) (layer "B.Cu") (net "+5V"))
 (segment (start 39.54 35) (end 61 35) (width 1) (layer "B.Cu") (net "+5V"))
 (segment (start 40.797918 52.797918) (end 41.595836 52) (width 1) (layer "B.Cu") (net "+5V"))
 (segment (start 36.704164 60.704164) (end 36 60) (width 1) (layer "B.Cu") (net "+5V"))
 (segment (start 36 74.54) (end 33.54 74.54) (width 1) (layer "B.Cu") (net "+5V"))
 (segment (start 56.73 61) (end 53 57.27) (width 1) (layer "B.Cu") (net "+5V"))
 (segment (start 33 55) (end 37 55) (width 1) (layer "B.Cu") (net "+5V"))
 (segment (start 40.797918 52.797918) (end 35 47) (width 1) (layer "B.Cu") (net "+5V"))
 (segment (start 43 64) (end 40.7 61.7) (width 1) (layer "B.Cu") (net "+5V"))
 (segment (start 40 52) (end 40.797918 52.797918) (width 1) (layer "B.Cu") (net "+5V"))
 (segment (start 65.998246 37.998246) (end 63 35) (width 1) (layer "B.Cu") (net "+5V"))
 (segment (start 35 39.54) (end 39 35.54) (width 1) (layer "B.Cu") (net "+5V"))
 (segment (start 71.023996 31) (end 77 31) (width 1) (layer "B.Cu") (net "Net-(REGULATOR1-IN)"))
 (segment (start 69.10575 32.918246) (end 71.023996 31) (width 1) (layer "B.Cu") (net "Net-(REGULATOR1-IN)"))
 (segment (start 79 39.08) (end 82 42.08) (width 1) (layer "B.Cu") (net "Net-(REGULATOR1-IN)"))
 (segment (start 79 34) (end 79 39.08) (width 1) (layer "B.Cu") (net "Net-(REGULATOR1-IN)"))
 (segment (start 77 34) (end 77 31) (width 1) (layer "B.Cu") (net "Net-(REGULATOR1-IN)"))
 (segment (start 77 34) (end 79 34) (width 1) (layer "B.Cu") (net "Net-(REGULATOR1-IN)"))
 (segment (start 53 52.19) (end 57.31 52.19) (width 1) (layer "B.Cu") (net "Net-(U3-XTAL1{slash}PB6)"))
 (segment (start 60 54.88) (end 64.12 54.88) (width 1) (layer "B.Cu") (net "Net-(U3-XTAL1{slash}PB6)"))
 (segment (start 64.12 54.88) (end 65 54) (width 1) (layer "B.Cu") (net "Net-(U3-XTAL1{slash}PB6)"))
 (segment (start 57.31 52.19) (end 60 54.88) (width 1) (layer "B.Cu") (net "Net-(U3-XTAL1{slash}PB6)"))
 (segment (start 53 49.65) (end 59.65 49.65) (width 1) (layer "B.Cu") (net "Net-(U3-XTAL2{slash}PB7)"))
 (segment (start 59.65 49.65) (end 60 50) (width 1) (layer "B.Cu") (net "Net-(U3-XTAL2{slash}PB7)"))
 (segment (start 60 50) (end 65 50) (width 1) (layer "B.Cu") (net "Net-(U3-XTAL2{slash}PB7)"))
 (segment (start 40.41 49.65) (end 45.38 49.65) (width 1) (layer "B.Cu") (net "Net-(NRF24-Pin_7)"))
 (segment (start 39 48.24) (end 40.41 49.65) (width 1) (layer "B.Cu") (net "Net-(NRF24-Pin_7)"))
 (segment (start 40.41 44.57) (end 45.38 44.57) (width 1) (layer "B.Cu") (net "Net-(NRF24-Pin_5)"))
 (segment (start 39 43.16) (end 40.41 44.57) (width 1) (layer "B.Cu") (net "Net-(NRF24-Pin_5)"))
 (segment (start 39 40.62) (end 40.41 42.03) (width 1) (layer "B.Cu") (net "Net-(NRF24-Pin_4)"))
 (segment (start 40.41 42.03) (end 45.38 42.03) (width 1) (layer "B.Cu") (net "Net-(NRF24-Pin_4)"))
 (segment (start 39 45.7) (end 40.41 47.11) (width 1) (layer "B.Cu") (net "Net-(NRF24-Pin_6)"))
 (segment (start 40.41 47.11) (end 45.38 47.11) (width 1) (layer "B.Cu") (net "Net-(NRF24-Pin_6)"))
 (segment (start 40.41 39.49) (end 45.38 39.49) (width 1) (layer "B.Cu") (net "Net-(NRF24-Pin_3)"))
 (segment (start 39 38.08) (end 40.41 39.49) (width 1) (layer "B.Cu") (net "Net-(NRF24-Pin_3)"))
 (segment (start 54.08 77) (end 54.08 73.59) (width 1) (layer "B.Cu") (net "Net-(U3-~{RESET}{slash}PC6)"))
 (segment (start 57.74 72.51) (end 57.75 72.5) (width 1) (layer "B.Cu") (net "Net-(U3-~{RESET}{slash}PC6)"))
 (segment (start 53 72.51) (end 57.74 72.51) (width 1) (layer "B.Cu") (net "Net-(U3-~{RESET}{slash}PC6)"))
 (segment (start 54.08 73.59) (end 53 72.51) (width 1) (layer "B.Cu") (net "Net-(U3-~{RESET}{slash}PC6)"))
 (segment (start 82 32.415534) (end 85.562233 35.977767) (width 1) (layer "B.Cu") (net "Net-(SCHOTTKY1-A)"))
 (segment (start 82 31.92) (end 82 32.415534) (width 1) (layer "B.Cu") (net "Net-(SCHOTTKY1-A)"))
 (segment (start 53 67.43) (end 53.77 68.2) (width 1) (layer "B.Cu") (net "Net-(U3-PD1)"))
 (segment (start 64 82) (end 39 82) (width 1) (layer "B.Cu") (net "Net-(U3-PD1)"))
 (segment (start 53.77 68.2) (end 64 68.2) (width 1) (layer "B.Cu") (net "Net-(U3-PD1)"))
 (segment (start 39 82) (end 39 75) (width 1) (layer "B.Cu") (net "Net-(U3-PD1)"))
 (segment (start 64 68.2) (end 64 82) (width 1) (layer "B.Cu") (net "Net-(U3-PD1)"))
 (segment (start 39 75) (end 36 72) (width 1) (layer "B.Cu") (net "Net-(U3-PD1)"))
 (segment (start 62 79) (end 62 72) (width 1) (layer "B.Cu") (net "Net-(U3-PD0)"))
 (segment (start 41 79) (end 42 80) (width 1) (layer "B.Cu") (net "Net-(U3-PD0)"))
 (segment (start 42 80) (end 61 80) (width 1) (layer "B.Cu") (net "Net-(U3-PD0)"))
 (segment (start 59.97 69.97) (end 53 69.97) (width 1) (layer "B.Cu") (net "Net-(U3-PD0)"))
 (segment (start 61 80) (end 62 79) (width 1) (layer "B.Cu") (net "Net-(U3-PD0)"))
 (segment (start 52.439898 69.97) (end 53 69.97) (width 1) (layer "B.Cu") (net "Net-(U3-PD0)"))
 (segment (start 41 74.46) (end 41 79) (width 1) (layer "B.Cu") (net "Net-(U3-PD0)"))
 (segment (start 36 69.46) (end 41 74.46) (width 1) (layer "B.Cu") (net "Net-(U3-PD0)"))
 (segment (start 62 72) (end 59.97 69.97) (width 1) (layer "B.Cu") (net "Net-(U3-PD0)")))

